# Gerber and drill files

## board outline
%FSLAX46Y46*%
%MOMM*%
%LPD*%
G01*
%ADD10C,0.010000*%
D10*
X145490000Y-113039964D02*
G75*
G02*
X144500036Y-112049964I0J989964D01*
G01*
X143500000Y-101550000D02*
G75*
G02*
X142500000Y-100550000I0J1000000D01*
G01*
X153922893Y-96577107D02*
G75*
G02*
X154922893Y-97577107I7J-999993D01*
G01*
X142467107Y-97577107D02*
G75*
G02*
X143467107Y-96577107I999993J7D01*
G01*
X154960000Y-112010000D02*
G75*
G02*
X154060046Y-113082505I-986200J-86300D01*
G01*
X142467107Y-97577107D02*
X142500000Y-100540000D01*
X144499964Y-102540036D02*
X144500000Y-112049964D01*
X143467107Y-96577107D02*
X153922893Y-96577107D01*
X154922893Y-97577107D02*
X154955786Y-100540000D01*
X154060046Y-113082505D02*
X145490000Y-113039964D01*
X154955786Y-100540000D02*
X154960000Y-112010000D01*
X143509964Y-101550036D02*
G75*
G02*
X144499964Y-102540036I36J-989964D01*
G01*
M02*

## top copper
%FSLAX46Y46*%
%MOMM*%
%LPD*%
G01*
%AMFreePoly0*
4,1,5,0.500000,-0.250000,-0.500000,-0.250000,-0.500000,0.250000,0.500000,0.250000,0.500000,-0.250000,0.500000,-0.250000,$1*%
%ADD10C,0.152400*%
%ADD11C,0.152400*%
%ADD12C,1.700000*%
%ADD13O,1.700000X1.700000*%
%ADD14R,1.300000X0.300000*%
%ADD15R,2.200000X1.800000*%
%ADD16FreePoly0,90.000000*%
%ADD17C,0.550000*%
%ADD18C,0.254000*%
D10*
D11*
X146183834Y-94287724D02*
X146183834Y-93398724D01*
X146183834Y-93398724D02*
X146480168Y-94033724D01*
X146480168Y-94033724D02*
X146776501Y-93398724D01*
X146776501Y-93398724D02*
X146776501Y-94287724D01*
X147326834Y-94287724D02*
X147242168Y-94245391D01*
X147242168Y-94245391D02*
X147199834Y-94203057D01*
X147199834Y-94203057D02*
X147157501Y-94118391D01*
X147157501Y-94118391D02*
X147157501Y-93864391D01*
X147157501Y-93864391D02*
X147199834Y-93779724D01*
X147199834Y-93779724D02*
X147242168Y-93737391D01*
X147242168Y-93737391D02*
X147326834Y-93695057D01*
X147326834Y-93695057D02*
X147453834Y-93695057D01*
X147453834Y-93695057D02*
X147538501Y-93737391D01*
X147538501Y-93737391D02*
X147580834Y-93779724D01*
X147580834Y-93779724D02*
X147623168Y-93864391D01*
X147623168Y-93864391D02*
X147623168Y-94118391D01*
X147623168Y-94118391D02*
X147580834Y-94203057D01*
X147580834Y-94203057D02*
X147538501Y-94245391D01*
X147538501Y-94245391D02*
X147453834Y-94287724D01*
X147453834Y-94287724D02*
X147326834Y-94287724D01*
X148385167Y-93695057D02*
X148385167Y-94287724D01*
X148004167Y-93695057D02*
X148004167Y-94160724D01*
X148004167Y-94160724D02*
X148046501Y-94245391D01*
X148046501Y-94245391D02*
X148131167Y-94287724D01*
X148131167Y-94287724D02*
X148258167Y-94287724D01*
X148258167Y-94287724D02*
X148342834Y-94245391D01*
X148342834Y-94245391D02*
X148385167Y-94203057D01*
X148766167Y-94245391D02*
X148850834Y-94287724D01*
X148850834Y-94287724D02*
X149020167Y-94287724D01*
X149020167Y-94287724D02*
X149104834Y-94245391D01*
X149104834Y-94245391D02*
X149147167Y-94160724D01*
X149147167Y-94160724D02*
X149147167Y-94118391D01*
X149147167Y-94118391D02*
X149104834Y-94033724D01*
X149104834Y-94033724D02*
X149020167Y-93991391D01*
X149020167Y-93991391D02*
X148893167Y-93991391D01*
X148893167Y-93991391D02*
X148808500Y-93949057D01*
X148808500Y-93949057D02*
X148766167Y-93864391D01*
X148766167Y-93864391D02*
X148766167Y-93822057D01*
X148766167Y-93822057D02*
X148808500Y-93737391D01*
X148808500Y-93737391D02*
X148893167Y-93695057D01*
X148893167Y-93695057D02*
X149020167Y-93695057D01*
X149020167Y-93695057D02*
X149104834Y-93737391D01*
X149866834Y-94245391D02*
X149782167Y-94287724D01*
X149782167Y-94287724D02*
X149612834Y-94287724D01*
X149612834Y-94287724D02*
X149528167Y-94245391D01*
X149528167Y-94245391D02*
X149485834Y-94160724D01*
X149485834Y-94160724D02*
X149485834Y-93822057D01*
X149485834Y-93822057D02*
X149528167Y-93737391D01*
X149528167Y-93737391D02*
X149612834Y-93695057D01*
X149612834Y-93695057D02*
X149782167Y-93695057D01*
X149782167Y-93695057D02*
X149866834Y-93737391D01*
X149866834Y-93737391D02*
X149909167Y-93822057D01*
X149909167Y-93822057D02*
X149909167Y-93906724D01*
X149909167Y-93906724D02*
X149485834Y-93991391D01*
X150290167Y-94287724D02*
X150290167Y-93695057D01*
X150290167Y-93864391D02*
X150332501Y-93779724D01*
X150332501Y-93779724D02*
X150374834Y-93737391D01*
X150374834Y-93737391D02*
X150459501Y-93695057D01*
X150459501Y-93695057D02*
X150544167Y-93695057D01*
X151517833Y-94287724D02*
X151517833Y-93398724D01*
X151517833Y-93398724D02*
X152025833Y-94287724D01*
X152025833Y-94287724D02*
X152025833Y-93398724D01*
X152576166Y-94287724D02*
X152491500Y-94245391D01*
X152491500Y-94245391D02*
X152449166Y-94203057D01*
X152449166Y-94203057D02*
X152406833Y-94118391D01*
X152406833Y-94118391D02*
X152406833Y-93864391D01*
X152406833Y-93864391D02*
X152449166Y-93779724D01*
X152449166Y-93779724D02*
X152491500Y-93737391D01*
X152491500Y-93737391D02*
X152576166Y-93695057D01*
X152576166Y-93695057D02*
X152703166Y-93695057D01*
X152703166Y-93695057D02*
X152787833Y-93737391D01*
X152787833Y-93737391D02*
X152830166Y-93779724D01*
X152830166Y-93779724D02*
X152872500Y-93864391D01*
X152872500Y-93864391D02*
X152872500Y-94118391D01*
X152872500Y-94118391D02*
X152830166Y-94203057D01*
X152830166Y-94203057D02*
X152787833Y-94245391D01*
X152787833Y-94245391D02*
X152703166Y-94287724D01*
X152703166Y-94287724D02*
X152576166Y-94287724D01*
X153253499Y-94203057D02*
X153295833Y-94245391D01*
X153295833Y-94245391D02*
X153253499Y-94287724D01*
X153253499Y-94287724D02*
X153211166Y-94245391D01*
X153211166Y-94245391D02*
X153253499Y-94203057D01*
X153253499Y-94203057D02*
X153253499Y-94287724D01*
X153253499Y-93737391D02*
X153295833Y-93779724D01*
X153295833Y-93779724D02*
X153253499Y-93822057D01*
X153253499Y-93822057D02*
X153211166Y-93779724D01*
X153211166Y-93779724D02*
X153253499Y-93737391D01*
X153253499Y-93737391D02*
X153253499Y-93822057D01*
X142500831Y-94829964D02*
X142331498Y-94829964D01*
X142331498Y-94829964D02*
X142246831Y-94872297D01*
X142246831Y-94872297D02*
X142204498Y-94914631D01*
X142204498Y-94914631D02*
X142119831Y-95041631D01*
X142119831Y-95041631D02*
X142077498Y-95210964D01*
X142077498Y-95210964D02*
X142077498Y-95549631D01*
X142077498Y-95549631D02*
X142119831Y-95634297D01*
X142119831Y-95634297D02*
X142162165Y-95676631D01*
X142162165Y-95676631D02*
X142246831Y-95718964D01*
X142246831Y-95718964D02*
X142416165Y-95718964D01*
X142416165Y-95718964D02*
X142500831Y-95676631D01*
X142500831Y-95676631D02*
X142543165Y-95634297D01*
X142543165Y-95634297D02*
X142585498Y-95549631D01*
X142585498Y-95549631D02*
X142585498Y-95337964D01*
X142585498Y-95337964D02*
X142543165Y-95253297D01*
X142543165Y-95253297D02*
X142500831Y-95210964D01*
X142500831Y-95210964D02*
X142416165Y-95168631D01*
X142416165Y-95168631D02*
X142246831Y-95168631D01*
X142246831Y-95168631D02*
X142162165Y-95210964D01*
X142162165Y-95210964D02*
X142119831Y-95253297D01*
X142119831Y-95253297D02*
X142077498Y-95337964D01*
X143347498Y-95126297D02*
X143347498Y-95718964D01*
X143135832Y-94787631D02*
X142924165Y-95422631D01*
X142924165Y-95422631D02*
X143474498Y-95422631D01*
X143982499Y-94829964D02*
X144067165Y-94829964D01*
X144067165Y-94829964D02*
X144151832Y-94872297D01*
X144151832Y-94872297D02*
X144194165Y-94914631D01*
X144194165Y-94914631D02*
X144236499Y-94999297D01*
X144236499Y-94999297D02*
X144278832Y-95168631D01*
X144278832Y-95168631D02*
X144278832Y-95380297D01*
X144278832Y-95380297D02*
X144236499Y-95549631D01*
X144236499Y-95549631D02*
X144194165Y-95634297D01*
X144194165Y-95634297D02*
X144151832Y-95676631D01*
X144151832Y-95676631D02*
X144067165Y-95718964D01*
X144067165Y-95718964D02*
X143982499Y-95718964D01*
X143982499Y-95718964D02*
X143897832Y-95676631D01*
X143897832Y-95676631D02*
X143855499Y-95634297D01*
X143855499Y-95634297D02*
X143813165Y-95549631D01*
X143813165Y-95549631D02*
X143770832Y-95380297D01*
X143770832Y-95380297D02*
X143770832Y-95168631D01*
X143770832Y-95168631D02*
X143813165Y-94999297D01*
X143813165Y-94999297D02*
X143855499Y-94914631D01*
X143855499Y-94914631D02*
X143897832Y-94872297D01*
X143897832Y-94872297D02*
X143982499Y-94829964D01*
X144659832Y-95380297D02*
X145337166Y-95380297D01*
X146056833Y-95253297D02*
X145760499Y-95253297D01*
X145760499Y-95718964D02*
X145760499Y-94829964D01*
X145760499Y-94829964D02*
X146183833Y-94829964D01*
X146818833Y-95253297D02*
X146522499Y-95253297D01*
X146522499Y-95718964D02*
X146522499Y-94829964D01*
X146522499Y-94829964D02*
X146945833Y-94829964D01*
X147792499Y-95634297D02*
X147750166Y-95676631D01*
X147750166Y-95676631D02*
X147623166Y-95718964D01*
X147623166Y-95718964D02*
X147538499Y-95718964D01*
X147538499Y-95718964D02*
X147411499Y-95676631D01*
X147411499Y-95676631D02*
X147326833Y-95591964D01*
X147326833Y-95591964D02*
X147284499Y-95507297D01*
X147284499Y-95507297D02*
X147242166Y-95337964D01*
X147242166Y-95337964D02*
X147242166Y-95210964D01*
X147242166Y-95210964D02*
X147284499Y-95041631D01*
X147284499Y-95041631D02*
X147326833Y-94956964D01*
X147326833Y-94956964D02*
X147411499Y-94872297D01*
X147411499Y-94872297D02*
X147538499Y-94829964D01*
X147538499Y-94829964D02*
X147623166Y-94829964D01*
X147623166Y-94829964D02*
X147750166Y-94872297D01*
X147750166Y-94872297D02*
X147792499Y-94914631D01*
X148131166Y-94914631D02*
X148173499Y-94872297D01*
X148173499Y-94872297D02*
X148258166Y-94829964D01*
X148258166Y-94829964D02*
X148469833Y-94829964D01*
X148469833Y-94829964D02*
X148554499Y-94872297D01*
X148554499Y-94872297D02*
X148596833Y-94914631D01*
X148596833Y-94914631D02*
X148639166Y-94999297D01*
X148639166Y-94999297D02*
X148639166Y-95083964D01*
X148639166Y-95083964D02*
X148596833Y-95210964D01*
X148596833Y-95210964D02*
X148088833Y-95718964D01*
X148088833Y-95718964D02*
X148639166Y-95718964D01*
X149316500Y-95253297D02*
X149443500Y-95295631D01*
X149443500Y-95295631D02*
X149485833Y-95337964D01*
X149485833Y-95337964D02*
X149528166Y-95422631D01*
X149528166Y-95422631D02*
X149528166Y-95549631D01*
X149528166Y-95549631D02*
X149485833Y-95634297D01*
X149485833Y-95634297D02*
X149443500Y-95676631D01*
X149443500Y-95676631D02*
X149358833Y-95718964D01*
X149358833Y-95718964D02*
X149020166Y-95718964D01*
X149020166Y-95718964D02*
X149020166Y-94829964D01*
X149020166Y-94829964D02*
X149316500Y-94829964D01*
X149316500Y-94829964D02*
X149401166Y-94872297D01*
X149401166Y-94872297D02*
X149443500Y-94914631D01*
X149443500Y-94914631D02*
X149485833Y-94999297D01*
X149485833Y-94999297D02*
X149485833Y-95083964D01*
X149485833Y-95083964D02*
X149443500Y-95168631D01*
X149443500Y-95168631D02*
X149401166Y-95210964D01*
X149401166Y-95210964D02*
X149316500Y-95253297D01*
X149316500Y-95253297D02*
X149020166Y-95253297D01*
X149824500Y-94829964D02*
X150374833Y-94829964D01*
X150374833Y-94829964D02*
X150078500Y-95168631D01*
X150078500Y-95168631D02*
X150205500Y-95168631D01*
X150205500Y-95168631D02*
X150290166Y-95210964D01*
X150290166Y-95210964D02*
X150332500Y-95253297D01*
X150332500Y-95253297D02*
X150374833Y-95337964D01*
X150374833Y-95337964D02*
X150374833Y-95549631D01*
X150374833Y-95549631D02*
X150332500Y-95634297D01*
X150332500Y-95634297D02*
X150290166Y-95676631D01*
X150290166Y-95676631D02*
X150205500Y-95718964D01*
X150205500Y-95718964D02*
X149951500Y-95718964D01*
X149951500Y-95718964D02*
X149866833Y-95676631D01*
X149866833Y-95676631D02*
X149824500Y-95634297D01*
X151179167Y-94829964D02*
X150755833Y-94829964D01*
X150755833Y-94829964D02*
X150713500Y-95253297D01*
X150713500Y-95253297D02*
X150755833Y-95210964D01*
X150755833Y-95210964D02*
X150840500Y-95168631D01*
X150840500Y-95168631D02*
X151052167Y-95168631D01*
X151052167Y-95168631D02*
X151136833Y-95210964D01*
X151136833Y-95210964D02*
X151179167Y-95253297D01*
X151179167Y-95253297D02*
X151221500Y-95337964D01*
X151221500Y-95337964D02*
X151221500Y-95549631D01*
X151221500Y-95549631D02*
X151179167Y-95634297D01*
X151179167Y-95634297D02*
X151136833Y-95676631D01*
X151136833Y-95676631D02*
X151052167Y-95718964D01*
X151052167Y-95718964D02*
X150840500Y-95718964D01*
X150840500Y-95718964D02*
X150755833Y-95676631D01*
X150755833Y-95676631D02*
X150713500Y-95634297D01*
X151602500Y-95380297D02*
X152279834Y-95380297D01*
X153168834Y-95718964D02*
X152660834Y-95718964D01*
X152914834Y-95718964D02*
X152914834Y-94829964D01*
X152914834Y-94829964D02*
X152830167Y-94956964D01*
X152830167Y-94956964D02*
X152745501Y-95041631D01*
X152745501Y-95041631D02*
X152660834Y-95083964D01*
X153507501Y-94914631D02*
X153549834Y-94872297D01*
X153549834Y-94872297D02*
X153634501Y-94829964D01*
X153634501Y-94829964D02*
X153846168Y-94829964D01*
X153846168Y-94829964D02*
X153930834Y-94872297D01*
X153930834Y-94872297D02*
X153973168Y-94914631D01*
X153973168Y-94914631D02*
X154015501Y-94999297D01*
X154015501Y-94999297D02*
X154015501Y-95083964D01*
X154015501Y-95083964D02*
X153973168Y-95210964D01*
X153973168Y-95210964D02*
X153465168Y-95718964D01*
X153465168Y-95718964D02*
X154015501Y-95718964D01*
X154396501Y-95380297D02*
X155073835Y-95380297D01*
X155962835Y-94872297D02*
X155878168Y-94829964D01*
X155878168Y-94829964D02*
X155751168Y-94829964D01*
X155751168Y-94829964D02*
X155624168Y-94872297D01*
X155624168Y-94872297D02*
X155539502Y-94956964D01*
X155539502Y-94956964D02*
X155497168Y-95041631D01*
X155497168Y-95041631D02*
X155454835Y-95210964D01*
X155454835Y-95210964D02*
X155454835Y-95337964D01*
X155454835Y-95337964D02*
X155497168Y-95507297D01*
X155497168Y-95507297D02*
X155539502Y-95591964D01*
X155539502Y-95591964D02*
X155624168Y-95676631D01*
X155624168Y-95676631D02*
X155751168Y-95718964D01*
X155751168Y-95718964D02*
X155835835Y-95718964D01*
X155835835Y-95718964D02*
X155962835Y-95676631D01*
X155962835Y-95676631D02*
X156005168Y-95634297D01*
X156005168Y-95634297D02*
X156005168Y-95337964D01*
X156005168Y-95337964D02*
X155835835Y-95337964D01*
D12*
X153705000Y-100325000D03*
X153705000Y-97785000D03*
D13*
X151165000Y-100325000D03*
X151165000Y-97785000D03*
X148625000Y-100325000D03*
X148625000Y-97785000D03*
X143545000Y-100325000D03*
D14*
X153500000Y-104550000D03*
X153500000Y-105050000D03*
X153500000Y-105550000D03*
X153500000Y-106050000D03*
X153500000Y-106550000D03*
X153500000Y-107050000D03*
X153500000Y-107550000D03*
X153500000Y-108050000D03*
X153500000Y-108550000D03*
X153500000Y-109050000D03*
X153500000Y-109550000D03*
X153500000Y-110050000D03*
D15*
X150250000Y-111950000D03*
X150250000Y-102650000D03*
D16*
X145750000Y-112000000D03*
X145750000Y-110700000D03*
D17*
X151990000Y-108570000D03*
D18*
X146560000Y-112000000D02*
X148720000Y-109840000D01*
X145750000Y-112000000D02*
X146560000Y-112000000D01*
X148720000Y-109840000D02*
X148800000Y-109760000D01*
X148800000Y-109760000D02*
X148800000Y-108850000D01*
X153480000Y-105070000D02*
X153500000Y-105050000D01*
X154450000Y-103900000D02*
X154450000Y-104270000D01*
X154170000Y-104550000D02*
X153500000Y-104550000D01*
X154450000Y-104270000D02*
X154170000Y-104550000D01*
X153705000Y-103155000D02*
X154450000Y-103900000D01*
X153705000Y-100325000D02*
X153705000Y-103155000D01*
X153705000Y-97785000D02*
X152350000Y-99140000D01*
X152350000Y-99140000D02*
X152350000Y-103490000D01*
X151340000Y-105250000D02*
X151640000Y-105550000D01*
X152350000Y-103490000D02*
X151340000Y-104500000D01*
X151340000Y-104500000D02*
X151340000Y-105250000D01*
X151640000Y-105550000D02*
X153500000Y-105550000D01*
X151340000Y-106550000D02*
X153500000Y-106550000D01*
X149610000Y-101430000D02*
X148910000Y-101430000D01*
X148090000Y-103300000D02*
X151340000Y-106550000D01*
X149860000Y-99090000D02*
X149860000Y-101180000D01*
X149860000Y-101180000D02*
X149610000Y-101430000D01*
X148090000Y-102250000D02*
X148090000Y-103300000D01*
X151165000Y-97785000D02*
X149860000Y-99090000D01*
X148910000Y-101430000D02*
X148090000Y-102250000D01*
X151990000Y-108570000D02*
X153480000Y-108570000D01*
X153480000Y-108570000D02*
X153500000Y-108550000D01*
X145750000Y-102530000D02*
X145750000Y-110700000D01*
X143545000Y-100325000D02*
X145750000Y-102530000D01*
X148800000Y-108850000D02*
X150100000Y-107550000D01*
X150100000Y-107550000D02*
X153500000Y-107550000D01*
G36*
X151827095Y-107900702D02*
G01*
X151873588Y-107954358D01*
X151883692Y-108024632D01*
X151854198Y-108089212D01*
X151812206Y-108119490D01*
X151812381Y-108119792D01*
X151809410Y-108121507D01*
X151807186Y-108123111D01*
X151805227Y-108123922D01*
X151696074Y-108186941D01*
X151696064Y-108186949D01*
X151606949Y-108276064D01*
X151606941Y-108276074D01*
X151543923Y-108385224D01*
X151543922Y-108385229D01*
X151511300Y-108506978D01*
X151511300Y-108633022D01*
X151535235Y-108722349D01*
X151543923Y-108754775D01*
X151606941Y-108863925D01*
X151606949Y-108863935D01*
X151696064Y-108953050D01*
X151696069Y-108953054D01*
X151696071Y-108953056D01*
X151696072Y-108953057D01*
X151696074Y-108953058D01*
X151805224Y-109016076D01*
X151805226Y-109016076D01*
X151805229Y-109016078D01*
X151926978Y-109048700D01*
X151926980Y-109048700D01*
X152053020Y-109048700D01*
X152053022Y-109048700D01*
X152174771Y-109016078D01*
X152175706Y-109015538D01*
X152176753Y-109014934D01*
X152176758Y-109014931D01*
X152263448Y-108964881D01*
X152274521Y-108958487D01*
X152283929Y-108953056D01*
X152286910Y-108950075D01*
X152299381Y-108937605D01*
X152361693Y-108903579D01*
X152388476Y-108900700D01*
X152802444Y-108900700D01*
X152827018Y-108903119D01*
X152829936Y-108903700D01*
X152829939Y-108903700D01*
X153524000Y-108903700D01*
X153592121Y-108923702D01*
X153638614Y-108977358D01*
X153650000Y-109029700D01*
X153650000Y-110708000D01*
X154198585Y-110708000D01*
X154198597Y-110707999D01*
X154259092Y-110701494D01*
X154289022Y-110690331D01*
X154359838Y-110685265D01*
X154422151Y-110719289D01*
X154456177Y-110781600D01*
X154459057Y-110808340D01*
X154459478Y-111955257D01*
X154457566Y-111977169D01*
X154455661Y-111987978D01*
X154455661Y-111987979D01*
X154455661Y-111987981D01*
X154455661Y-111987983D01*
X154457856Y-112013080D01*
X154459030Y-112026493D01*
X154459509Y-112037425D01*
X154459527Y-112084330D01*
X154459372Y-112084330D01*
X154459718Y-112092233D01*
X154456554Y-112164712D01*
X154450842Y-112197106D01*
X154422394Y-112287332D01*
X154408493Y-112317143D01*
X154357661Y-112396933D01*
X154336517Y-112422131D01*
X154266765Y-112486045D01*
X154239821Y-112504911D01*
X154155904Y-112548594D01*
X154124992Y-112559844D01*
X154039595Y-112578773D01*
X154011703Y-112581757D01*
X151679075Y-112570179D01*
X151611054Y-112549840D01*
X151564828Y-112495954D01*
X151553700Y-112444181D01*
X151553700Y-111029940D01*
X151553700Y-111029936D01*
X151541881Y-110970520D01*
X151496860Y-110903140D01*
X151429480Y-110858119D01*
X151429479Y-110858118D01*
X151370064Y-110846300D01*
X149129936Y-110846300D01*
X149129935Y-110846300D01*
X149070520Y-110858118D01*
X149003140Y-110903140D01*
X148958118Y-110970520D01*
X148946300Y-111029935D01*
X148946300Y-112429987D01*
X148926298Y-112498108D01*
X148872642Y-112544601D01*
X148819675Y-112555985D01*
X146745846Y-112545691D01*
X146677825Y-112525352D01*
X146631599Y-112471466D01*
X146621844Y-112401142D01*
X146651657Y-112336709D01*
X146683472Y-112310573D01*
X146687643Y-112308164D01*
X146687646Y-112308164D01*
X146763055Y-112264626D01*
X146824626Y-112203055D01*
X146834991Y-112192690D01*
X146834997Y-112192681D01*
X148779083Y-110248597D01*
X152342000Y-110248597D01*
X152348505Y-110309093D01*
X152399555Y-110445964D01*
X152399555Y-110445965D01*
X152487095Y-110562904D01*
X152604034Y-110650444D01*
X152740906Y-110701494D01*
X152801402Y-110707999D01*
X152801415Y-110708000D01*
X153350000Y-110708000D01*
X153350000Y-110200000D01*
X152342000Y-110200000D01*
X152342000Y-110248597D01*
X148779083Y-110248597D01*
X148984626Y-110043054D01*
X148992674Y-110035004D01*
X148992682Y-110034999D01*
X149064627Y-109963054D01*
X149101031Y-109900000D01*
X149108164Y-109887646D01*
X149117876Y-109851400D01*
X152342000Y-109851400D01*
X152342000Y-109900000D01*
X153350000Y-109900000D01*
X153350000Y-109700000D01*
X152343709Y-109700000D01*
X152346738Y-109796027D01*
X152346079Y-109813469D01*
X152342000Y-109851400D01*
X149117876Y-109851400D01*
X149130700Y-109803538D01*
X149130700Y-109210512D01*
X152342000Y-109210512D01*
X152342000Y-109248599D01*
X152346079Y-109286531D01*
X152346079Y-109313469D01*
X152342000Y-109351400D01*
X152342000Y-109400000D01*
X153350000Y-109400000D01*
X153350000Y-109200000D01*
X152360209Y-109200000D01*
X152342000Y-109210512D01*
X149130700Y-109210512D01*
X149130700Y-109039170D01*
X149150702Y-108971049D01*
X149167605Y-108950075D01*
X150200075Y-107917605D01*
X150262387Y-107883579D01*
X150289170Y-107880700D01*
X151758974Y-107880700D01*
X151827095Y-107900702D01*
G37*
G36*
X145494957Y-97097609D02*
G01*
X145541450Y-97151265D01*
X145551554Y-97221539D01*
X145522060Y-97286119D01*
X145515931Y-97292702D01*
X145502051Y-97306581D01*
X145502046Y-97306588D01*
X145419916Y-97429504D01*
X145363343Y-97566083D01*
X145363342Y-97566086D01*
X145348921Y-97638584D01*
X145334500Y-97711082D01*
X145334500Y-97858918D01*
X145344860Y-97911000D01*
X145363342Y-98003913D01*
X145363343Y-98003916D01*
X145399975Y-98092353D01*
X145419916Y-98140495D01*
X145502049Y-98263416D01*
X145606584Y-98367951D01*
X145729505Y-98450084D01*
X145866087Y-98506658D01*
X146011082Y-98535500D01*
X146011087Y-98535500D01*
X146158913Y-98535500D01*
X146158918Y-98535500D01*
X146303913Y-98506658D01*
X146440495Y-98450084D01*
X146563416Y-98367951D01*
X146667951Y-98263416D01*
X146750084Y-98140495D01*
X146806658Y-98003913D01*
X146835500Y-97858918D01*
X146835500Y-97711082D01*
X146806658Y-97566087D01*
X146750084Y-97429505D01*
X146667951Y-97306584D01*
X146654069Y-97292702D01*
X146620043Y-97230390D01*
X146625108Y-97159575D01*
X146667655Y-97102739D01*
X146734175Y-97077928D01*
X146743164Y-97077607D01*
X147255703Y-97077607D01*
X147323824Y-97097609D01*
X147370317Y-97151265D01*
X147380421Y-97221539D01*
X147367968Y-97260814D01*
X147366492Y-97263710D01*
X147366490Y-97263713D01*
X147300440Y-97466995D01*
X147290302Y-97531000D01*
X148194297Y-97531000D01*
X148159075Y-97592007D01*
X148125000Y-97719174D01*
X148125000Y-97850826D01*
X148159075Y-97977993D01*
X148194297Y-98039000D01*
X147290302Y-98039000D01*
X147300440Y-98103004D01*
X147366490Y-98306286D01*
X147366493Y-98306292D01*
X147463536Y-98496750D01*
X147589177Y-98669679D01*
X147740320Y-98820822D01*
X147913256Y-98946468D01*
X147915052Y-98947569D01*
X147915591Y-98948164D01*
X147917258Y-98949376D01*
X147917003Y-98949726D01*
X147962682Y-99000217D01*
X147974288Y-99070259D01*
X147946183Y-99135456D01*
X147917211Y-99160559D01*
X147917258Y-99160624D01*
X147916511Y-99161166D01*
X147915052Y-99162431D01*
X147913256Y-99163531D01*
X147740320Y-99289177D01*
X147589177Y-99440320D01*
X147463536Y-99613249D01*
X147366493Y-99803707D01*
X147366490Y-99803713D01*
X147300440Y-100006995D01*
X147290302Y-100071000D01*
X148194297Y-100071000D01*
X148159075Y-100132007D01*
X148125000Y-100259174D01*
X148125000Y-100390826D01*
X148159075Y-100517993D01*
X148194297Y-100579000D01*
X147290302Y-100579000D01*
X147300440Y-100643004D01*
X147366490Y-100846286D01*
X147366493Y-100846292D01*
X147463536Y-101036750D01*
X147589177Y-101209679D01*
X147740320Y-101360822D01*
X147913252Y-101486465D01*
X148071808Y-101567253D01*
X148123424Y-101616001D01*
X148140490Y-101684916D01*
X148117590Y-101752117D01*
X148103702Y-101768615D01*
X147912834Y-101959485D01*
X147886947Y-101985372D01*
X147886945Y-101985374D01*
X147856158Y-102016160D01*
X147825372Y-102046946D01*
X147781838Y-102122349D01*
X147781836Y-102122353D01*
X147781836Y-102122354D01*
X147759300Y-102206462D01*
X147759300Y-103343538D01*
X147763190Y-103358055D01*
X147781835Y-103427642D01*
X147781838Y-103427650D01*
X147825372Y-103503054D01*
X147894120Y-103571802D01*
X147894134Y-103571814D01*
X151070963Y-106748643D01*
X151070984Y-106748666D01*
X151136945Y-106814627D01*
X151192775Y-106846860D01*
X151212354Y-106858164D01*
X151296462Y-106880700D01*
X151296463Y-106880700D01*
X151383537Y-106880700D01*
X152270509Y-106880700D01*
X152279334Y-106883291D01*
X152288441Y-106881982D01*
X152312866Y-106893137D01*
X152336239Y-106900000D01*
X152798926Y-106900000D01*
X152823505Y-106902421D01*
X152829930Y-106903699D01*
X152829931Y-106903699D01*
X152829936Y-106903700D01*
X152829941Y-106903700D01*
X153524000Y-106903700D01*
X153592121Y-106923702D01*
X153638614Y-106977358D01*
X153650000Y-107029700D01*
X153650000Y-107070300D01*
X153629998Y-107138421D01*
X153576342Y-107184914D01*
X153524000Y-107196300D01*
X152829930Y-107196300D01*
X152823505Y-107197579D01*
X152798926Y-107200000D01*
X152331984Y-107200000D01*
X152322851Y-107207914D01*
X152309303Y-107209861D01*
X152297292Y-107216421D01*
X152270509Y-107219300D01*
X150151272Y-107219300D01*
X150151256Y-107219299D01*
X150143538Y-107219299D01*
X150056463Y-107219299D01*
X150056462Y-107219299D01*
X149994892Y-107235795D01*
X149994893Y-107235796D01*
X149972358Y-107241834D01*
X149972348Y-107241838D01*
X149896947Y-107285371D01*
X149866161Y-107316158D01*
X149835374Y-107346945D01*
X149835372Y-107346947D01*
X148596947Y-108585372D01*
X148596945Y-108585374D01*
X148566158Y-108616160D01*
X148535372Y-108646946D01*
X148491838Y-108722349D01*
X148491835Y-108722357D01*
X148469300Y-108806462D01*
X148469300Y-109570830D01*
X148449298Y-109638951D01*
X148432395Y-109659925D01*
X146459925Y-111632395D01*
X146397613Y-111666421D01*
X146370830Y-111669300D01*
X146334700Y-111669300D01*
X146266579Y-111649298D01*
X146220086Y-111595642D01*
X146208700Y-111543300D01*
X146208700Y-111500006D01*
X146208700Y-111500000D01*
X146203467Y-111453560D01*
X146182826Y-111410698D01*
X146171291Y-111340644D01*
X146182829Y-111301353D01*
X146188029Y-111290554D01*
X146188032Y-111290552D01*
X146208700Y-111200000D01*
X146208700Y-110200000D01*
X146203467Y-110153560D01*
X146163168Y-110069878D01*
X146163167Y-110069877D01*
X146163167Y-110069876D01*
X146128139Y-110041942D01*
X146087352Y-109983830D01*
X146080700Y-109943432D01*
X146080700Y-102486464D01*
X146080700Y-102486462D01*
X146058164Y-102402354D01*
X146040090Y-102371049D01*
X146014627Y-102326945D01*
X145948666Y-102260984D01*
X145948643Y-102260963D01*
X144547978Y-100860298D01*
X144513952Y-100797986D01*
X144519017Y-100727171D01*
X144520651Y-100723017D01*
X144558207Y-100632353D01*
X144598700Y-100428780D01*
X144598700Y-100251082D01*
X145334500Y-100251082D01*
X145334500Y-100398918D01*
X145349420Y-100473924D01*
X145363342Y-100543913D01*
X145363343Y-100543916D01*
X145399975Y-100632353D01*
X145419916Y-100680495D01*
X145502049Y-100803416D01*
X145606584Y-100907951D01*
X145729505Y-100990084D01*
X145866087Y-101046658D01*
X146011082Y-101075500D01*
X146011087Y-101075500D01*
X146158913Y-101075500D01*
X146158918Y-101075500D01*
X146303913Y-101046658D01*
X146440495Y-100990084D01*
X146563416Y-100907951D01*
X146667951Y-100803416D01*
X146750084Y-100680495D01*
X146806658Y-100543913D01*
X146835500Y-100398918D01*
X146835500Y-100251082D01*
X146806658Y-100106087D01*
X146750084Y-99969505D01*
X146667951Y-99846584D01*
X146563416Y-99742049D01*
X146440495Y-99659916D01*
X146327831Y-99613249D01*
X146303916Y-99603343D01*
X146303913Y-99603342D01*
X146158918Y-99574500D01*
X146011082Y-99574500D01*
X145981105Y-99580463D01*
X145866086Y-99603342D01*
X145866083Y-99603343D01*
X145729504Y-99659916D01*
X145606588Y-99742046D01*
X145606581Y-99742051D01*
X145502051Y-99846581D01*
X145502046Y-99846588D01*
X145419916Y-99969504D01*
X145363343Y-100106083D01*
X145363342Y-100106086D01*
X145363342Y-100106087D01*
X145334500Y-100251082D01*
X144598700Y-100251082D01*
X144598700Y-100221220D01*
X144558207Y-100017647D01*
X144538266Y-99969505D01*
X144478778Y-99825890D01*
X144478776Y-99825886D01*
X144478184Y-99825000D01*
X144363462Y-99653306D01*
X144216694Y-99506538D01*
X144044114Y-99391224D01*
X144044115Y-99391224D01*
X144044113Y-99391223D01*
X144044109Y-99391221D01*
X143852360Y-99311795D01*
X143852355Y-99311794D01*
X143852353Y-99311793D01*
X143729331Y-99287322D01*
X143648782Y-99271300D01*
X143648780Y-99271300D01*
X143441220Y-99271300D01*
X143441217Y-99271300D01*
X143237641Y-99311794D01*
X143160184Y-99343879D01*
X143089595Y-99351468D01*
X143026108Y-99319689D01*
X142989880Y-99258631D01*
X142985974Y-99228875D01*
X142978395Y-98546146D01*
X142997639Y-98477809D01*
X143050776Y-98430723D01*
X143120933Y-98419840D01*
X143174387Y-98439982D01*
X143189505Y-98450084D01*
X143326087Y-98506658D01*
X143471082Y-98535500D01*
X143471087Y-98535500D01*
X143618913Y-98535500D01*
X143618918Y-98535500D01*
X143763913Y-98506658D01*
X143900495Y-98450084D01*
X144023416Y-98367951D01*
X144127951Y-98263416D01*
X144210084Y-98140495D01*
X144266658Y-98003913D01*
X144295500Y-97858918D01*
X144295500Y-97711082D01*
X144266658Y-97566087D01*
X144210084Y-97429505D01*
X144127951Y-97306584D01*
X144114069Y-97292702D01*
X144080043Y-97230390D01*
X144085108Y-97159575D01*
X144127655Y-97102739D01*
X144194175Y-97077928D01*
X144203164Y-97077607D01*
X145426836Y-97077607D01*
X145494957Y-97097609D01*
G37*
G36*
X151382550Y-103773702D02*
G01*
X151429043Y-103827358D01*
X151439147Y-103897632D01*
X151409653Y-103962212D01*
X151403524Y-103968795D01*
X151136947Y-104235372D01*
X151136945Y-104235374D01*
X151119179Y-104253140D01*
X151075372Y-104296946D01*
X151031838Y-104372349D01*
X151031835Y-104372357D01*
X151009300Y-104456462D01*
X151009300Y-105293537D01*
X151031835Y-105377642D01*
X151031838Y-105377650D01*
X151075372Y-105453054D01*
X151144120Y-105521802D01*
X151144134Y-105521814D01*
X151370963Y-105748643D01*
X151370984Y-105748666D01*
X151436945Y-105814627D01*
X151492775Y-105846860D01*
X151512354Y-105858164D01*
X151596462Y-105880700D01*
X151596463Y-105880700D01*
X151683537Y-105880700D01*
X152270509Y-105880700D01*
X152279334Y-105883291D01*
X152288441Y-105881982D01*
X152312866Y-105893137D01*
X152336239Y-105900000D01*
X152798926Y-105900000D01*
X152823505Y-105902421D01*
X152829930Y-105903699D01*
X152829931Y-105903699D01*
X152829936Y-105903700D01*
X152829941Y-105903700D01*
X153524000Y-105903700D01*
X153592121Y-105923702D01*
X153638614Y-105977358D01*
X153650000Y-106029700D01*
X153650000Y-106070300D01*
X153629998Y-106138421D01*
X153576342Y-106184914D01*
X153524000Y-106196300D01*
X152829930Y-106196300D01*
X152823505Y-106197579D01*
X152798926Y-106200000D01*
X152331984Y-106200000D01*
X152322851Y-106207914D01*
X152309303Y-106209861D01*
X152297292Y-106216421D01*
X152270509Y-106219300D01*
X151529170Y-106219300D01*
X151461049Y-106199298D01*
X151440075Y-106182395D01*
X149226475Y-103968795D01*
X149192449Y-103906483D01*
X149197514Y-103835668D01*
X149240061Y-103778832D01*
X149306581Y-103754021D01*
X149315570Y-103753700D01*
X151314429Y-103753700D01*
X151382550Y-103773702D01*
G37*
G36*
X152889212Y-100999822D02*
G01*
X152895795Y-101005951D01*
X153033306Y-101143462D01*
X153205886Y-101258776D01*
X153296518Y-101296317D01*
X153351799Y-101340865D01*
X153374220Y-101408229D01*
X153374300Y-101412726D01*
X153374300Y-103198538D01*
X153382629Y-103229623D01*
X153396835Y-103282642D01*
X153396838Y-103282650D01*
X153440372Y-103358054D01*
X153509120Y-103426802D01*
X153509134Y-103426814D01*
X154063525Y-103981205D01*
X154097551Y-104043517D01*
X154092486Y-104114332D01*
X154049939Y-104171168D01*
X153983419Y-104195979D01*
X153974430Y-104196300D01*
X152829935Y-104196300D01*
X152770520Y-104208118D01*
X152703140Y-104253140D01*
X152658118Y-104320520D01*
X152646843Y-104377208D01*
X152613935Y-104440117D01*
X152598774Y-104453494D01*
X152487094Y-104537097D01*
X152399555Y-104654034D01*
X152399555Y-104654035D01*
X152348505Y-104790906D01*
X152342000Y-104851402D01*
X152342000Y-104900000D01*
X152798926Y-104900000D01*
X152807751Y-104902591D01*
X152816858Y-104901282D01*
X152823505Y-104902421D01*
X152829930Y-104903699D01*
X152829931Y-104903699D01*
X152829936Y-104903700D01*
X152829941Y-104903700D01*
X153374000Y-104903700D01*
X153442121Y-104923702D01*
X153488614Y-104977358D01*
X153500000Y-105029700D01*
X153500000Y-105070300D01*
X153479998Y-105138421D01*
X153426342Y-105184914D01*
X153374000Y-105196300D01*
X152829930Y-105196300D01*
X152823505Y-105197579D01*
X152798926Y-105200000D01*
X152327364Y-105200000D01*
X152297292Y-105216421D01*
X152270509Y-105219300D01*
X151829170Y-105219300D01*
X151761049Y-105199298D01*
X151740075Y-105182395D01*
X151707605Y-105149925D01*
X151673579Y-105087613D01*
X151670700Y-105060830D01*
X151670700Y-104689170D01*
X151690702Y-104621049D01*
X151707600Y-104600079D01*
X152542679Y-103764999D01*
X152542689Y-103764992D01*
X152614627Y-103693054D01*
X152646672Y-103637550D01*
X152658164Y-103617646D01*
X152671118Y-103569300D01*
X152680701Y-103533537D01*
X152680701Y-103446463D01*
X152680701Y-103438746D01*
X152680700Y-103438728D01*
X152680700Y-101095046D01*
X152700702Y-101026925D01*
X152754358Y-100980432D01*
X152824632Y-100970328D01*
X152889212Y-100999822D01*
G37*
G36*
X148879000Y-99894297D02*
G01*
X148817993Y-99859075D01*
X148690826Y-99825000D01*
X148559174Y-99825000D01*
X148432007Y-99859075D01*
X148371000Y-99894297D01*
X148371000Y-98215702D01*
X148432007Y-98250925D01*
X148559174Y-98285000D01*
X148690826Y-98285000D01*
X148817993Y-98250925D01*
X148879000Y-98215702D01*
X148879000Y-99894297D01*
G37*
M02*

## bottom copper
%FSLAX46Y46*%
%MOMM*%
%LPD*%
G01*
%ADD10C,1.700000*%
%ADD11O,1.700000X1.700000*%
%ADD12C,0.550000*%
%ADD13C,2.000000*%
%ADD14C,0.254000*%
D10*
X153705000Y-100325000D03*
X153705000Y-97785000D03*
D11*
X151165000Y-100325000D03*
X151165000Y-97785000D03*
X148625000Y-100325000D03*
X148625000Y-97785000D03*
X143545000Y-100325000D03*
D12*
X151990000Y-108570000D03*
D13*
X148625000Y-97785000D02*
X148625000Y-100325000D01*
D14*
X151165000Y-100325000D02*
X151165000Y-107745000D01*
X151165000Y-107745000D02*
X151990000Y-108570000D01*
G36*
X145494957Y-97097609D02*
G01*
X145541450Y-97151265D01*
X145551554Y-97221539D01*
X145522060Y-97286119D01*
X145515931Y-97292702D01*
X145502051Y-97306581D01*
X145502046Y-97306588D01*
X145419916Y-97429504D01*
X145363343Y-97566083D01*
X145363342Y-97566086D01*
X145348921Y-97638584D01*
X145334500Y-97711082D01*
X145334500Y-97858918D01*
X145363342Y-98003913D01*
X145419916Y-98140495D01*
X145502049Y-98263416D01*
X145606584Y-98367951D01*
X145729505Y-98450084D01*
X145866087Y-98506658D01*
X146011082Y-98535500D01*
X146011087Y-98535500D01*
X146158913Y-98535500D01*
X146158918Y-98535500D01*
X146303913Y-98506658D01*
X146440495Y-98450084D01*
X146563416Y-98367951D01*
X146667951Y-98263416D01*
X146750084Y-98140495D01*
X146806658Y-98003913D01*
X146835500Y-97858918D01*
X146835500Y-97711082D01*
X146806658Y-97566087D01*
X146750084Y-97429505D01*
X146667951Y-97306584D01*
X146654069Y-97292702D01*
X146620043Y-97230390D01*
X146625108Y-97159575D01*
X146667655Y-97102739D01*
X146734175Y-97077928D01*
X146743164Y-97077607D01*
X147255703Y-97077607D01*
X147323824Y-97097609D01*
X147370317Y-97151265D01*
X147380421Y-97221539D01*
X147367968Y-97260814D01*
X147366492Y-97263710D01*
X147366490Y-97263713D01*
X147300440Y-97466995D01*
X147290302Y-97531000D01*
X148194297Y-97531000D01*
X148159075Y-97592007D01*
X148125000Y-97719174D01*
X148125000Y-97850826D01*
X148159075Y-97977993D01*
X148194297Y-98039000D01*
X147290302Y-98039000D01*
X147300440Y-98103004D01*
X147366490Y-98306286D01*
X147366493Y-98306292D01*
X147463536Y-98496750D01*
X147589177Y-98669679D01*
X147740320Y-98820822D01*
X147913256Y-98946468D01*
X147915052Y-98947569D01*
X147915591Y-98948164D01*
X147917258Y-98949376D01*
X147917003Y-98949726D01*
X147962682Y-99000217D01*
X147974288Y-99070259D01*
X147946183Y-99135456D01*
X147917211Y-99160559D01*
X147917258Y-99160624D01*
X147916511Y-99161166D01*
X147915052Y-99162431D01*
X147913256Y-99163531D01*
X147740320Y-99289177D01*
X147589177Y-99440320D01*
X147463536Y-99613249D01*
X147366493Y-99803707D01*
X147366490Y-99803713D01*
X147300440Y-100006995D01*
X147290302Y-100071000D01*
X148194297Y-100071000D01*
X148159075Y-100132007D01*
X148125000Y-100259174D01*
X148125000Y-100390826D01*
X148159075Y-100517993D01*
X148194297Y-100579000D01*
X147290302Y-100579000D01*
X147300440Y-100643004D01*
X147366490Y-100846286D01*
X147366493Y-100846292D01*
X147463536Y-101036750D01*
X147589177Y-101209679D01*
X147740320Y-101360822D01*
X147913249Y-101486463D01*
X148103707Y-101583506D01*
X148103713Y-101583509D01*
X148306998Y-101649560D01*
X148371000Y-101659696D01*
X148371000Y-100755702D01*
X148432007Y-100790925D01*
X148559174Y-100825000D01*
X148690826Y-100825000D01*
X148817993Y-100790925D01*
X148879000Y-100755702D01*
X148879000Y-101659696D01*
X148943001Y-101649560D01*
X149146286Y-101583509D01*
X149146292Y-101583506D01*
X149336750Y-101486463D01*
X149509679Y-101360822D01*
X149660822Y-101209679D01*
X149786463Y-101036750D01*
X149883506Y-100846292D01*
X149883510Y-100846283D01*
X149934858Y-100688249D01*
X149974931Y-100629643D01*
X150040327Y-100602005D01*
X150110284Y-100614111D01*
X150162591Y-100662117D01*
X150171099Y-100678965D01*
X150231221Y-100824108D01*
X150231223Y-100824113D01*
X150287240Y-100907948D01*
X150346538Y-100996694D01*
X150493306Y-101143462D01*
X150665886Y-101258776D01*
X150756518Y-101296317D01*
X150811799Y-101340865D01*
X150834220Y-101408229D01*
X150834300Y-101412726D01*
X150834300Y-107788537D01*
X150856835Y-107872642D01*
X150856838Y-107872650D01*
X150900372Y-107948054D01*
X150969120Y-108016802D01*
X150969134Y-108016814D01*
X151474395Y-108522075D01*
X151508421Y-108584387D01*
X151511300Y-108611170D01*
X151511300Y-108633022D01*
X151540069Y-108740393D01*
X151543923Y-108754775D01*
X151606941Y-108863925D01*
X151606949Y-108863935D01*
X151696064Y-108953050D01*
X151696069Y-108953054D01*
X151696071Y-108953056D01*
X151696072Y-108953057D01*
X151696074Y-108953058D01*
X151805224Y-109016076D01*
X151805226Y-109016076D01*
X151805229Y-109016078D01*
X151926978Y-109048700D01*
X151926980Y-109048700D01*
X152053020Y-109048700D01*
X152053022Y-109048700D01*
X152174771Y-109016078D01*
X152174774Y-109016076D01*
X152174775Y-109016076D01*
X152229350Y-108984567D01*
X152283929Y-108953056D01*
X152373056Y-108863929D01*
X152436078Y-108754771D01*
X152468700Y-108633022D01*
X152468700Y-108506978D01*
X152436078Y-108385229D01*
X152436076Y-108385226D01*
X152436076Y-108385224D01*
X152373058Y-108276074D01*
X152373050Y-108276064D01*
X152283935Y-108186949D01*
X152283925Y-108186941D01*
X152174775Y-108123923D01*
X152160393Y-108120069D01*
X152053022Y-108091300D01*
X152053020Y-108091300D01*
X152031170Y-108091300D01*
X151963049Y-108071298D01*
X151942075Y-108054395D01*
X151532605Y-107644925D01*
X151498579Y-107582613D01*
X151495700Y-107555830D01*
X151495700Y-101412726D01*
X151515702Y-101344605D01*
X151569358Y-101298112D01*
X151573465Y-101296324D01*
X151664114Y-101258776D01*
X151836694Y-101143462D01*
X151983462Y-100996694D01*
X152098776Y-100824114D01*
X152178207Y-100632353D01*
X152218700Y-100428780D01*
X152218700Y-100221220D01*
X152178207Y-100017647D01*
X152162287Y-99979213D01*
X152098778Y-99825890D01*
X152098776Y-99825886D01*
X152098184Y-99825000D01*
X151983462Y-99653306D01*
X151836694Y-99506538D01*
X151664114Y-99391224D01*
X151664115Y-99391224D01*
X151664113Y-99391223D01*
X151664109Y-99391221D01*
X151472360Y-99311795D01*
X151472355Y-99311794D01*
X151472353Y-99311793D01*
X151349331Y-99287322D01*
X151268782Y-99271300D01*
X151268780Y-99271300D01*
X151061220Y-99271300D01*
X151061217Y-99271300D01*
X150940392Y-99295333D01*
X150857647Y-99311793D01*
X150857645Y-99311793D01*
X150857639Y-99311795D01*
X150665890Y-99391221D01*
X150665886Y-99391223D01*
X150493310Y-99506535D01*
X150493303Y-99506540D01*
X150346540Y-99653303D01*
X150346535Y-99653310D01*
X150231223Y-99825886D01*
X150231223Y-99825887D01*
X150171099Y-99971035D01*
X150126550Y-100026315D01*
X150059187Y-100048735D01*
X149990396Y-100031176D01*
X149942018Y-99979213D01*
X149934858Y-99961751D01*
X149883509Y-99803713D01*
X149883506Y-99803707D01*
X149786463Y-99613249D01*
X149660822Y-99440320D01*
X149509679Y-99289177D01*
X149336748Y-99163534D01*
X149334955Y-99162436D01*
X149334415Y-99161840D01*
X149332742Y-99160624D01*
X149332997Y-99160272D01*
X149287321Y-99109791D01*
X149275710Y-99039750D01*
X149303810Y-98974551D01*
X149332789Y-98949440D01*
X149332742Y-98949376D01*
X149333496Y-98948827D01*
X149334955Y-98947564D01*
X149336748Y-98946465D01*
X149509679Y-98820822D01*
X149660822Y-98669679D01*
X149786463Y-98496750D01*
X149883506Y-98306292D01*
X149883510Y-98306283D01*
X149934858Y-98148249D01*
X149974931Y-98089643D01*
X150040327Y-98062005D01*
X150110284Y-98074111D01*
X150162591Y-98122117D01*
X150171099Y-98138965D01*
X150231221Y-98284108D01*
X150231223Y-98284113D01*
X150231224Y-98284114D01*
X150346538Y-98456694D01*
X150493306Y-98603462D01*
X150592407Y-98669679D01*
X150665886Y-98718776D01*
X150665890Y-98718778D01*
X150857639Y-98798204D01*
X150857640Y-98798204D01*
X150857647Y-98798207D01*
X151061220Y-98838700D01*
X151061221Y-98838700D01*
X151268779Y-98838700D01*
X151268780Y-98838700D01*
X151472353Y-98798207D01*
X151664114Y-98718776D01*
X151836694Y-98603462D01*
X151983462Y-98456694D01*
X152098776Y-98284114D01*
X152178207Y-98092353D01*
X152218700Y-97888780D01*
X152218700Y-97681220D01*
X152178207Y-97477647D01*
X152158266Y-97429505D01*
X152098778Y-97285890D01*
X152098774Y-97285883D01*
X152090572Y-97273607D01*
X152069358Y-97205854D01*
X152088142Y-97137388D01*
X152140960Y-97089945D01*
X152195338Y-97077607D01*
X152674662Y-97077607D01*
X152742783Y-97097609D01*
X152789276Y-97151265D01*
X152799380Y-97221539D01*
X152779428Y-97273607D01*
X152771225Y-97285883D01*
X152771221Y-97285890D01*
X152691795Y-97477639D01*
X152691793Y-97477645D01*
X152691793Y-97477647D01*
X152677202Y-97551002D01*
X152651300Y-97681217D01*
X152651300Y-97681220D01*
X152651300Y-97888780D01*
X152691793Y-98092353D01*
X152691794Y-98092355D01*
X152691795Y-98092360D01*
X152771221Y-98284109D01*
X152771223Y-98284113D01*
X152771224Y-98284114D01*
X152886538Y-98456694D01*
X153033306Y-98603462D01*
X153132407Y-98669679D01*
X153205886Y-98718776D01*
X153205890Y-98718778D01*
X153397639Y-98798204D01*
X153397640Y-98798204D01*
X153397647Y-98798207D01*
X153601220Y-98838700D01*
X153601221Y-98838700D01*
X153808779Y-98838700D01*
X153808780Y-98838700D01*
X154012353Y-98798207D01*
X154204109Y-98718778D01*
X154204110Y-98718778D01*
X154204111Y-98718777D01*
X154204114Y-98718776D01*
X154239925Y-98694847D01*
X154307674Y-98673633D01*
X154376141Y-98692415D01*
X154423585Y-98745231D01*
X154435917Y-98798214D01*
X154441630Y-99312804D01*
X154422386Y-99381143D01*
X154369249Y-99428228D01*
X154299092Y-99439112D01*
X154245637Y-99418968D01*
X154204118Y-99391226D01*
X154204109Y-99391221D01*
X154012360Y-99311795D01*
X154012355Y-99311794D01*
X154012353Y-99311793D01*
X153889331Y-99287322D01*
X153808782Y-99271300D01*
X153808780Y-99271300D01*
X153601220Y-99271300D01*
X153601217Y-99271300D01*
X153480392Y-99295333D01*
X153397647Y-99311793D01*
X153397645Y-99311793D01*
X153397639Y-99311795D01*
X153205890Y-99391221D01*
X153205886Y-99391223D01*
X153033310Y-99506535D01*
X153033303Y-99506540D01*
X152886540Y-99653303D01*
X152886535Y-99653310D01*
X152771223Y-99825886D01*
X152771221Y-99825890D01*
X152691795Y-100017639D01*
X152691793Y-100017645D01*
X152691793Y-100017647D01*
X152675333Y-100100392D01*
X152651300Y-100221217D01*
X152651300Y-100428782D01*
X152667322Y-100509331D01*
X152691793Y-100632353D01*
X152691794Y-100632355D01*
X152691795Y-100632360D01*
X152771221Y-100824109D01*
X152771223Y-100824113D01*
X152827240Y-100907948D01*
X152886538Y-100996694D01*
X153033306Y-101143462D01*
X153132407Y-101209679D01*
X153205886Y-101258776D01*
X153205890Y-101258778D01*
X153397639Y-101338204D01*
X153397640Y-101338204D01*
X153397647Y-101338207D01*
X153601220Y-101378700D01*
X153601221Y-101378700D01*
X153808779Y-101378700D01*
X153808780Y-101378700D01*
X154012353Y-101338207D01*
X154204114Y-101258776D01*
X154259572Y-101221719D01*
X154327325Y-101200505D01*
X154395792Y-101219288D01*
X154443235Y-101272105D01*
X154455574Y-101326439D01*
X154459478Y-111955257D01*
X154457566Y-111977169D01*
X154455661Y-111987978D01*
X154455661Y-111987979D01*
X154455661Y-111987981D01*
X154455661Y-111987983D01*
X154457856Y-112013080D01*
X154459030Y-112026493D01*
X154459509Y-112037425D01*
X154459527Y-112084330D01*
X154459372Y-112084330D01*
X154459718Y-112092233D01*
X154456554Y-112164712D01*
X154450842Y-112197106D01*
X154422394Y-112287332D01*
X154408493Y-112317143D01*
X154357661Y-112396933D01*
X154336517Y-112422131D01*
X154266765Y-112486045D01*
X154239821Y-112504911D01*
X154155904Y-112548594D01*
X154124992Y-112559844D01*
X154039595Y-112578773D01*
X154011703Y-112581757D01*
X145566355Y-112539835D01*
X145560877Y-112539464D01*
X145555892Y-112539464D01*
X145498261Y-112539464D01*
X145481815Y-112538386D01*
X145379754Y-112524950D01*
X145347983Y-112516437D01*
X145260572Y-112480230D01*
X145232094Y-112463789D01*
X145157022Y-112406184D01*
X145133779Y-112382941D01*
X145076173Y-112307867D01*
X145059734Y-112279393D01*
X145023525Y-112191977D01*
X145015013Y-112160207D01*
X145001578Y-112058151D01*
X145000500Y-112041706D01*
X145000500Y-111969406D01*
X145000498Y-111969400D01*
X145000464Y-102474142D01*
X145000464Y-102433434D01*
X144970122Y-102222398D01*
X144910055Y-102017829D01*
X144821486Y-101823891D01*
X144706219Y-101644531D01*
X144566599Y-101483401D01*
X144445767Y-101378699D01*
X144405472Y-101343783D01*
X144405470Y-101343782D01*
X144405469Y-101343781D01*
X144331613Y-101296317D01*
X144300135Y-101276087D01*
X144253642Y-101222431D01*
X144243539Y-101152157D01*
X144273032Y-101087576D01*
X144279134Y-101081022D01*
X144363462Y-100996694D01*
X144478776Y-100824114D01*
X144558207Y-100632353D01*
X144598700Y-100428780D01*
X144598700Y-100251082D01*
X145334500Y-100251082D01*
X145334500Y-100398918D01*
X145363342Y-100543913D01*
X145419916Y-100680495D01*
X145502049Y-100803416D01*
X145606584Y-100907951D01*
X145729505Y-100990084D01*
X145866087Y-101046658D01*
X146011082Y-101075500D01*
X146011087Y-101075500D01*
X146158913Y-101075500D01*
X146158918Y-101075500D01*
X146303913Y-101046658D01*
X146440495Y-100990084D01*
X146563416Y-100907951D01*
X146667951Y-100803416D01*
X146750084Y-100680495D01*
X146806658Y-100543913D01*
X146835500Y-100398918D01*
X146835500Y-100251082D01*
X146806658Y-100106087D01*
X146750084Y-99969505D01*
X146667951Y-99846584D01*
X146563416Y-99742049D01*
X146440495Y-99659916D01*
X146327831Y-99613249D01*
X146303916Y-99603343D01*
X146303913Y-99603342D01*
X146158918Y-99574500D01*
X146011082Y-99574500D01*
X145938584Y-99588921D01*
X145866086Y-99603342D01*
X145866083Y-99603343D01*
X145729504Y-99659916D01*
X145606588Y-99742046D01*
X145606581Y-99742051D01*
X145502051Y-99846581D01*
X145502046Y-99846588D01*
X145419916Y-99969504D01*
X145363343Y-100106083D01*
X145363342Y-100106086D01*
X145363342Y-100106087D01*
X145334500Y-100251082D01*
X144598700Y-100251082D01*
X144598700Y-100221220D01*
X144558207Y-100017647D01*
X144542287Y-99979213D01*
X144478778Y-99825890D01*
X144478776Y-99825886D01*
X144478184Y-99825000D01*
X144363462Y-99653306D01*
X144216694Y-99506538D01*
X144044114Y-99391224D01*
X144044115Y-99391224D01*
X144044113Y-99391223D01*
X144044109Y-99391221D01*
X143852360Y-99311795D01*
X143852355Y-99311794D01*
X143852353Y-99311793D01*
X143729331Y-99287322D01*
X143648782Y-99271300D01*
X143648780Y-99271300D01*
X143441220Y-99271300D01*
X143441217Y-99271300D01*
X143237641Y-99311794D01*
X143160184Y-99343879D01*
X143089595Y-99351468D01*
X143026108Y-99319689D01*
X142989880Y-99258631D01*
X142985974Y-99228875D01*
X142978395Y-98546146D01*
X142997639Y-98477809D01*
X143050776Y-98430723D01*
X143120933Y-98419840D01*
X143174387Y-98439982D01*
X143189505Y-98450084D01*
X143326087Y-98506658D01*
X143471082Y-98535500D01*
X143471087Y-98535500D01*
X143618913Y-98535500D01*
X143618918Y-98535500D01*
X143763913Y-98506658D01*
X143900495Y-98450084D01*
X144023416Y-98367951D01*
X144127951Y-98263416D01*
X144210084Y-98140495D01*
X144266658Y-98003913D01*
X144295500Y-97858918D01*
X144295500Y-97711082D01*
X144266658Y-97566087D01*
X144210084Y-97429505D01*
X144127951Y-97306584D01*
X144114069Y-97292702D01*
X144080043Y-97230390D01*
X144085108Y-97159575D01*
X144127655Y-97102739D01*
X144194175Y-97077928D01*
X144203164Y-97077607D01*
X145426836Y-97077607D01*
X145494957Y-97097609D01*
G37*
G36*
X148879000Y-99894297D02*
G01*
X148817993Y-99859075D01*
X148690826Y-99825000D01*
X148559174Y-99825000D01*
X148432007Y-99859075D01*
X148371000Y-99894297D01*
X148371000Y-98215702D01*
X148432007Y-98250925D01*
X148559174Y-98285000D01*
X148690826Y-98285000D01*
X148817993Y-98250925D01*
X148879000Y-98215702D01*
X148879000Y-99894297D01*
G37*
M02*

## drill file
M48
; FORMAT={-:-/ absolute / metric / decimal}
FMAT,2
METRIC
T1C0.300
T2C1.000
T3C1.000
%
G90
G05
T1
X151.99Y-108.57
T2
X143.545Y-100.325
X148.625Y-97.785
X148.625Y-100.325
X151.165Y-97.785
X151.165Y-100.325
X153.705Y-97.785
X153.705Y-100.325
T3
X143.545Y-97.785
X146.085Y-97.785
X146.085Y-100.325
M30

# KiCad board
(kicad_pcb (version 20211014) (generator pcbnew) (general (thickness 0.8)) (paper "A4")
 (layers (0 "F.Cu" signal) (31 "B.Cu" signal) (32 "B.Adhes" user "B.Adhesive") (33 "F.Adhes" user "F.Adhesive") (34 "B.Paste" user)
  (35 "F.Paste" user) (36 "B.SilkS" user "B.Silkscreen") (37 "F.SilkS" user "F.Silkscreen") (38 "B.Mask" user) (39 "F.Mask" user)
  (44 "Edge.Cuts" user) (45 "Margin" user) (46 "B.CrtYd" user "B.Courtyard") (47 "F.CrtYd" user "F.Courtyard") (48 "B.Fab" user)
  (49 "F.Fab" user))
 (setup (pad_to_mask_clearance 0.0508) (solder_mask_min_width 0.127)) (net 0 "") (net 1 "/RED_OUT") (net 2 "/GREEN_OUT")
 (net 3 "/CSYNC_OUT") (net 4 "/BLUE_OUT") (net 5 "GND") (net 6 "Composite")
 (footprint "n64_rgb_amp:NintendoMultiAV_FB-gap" (layer "F.Cu") (at 147.355 99.055)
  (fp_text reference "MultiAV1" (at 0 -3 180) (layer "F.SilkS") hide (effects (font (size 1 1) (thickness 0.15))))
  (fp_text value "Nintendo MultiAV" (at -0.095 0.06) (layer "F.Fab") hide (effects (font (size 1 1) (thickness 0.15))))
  (pad "" np_thru_hole circle (at -1.27 -1.27) (size 1 1) (drill 1) (layers *.Cu *.Mask))
  (pad "" np_thru_hole circle (at -3.81 -1.27) (size 1 1) (drill 1) (layers *.Cu *.Mask))
  (pad "" np_thru_hole oval (at -1.27 1.27) (size 1 1) (drill 1) (layers *.Cu *.Mask))
  (pad "1" thru_hole circle (at 6.35 1.27) (size 1.7 1.7) (drill 1) (layers *.Cu *.Mask) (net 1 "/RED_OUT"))
  (pad "2" thru_hole circle (at 6.35 -1.27) (size 1.7 1.7) (drill 1) (layers *.Cu *.Mask) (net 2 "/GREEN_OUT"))
  (pad "3" thru_hole oval (at 3.81 1.27) (size 1.7 1.7) (drill 1) (layers *.Cu *.Mask) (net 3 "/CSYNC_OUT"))
  (pad "4" thru_hole oval (at 3.81 -1.27) (size 1.7 1.7) (drill 1) (layers *.Cu *.Mask) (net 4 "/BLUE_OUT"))
  (pad "5" thru_hole oval (at 1.27 1.27) (size 1.7 1.7) (drill 1) (layers *.Cu *.Mask) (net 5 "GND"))
  (pad "6" thru_hole oval (at 1.27 -1.27) (size 1.7 1.7) (drill 1) (layers *.Cu *.Mask) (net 5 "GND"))
  (pad "10" thru_hole oval (at -3.81 1.27) (size 1.7 1.7) (drill 1) (layers *.Cu *.Mask) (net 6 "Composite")))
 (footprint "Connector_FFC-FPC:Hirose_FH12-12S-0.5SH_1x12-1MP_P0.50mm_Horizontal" (layer "F.Cu") (at 151.65 107.3 -90)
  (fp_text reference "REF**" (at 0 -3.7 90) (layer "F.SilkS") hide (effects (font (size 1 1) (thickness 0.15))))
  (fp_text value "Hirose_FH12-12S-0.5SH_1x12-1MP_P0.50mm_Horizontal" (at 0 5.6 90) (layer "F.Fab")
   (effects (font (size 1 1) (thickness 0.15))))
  (pad "1" smd rect (at -2.75 -1.85 270) (size 0.3 1.3) (layers "F.Cu" "F.Paste" "F.Mask"))
  (pad "2" smd rect (at -2.25 -1.85 270) (size 0.3 1.3) (layers "F.Cu" "F.Paste" "F.Mask") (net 5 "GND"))
  (pad "3" smd rect (at -1.75 -1.85 270) (size 0.3 1.3) (layers "F.Cu" "F.Paste" "F.Mask"))
  (pad "4" smd rect (at -1.25 -1.85 270) (size 0.3 1.3) (layers "F.Cu" "F.Paste" "F.Mask") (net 5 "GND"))
  (pad "5" smd rect (at -0.75 -1.85 270) (size 0.3 1.3) (layers "F.Cu" "F.Paste" "F.Mask"))
  (pad "6" smd rect (at -0.25 -1.85 270) (size 0.3 1.3) (layers "F.Cu" "F.Paste" "F.Mask") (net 5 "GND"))
  (pad "7" smd rect (at 0.25 -1.85 270) (size 0.3 1.3) (layers "F.Cu" "F.Paste" "F.Mask"))
  (pad "8" smd rect (at 0.75 -1.85 270) (size 0.3 1.3) (layers "F.Cu" "F.Paste" "F.Mask") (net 5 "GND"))
  (pad "9" smd rect (at 1.25 -1.85 270) (size 0.3 1.3) (layers "F.Cu" "F.Paste" "F.Mask"))
  (pad "10" smd rect (at 1.75 -1.85 270) (size 0.3 1.3) (layers "F.Cu" "F.Paste" "F.Mask") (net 5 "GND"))
  (pad "11" smd rect (at 2.25 -1.85 270) (size 0.3 1.3) (layers "F.Cu" "F.Paste" "F.Mask") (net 5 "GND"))
  (pad "12" smd rect (at 2.75 -1.85 270) (size 0.3 1.3) (layers "F.Cu" "F.Paste" "F.Mask") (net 5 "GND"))
  (pad "MP" smd rect (at 4.65 1.4 270) (size 1.8 2.2) (layers "F.Cu" "F.Paste" "F.Mask"))
  (pad "MP" smd rect (at -4.65 1.4 270) (size 1.8 2.2) (layers "F.Cu" "F.Paste" "F.Mask")))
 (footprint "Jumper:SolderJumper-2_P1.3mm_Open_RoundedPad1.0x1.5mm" (layer "F.Cu") (at 145.75 111.35 90)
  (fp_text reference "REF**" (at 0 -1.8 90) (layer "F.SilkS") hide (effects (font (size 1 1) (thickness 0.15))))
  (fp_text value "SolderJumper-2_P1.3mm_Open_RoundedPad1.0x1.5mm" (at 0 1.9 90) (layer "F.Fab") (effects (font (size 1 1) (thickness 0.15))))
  (pad "1" smd custom (at -0.65 0 90) (size 1 0.5) (layers "F.Cu" "F.Mask") (zone_connect 2) (options (clearance outline) (anchor rect))
   (primitives))
  (pad "2" smd custom (at 0.65 0 90) (size 1 0.5) (layers "F.Cu" "F.Mask") (zone_connect 2) (options (clearance outline) (anchor rect))
   (primitives)))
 (gr_arc (start 145.49 113.039964) (mid 144.789964 112.75) (end 144.5 112.049964) (layer "Edge.Cuts") (width 0.01))
 (gr_arc (start 143.5 101.55) (mid 142.792893 101.257107) (end 142.5 100.55) (layer "Edge.Cuts") (width 0.01))
 (gr_arc (start 153.922893 96.577107) (mid 154.63 96.87) (end 154.922893 97.577107) (layer "Edge.Cuts") (width 0.01))
 (gr_arc (start 142.467107 97.577107) (mid 142.76 96.87) (end 143.467107 96.577107) (layer "Edge.Cuts") (width 0.01))
 (gr_arc (start 154.96 112.01) (mid 154.732149 112.732644) (end 154.060046 113.082505) (layer "Edge.Cuts") (width 0.01))
 (gr_line (start 142.467107 97.577107) (end 142.5 100.54) (layer "Edge.Cuts") (width 0.01))
 (gr_line (start 144.499964 102.540036) (end 144.5 112.049964) (layer "Edge.Cuts") (width 0.01))
 (gr_line (start 143.467107 96.577107) (end 153.922893 96.577107) (layer "Edge.Cuts") (width 0.01))
 (gr_line (start 154.922893 97.577107) (end 154.955786 100.54) (layer "Edge.Cuts") (width 0.01))
 (gr_line (start 154.060046 113.082505) (end 145.49 113.039964) (layer "Edge.Cuts") (width 0.01))
 (gr_line (start 154.955786 100.54) (end 154.96 112.01) (layer "Edge.Cuts") (width 0.01))
 (gr_arc (start 143.509964 101.550036) (mid 144.21 101.84) (end 144.499964 102.540036) (layer "Edge.Cuts") (width 0.01))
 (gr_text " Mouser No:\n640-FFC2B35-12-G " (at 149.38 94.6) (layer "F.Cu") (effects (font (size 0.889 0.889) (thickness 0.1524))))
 (segment (start 146.56 112) (end 148.72 109.84) (width 0.254) (layer "F.Cu") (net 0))
 (segment (start 145.75 112) (end 146.56 112) (width 0.254) (layer "F.Cu") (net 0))
 (segment (start 148.72 109.84) (end 148.8 109.76) (width 0.254) (layer "F.Cu") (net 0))
 (segment (start 148.8 109.76) (end 148.8 108.85) (width 0.254) (layer "F.Cu") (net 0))
 (segment (start 153.48 105.07) (end 153.5 105.05) (width 0.254) (layer "F.Cu") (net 5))
 (segment (start 148.625 97.785) (end 148.625 100.325) (width 2) (layer "B.Cu") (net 5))
 (segment (start 154.45 103.9) (end 154.45 104.27) (width 0.254) (layer "F.Cu") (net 1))
 (segment (start 154.17 104.55) (end 153.5 104.55) (width 0.254) (layer "F.Cu") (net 1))
 (segment (start 154.45 104.27) (end 154.17 104.55) (width 0.254) (layer "F.Cu") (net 1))
 (segment (start 153.705 103.155) (end 154.45 103.9) (width 0.254) (layer "F.Cu") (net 1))
 (segment (start 153.705 100.325) (end 153.705 103.155) (width 0.254) (layer "F.Cu") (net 1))
 (segment (start 153.705 97.785) (end 152.35 99.14) (width 0.254) (layer "F.Cu") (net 2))
 (segment (start 152.35 99.14) (end 152.35 103.49) (width 0.254) (layer "F.Cu") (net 2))
 (segment (start 151.34 105.25) (end 151.64 105.55) (width 0.254) (layer "F.Cu") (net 2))
 (segment (start 152.35 103.49) (end 151.34 104.5) (width 0.254) (layer "F.Cu") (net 2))
 (segment (start 151.34 104.5) (end 151.34 105.25) (width 0.254) (layer "F.Cu") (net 2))
 (segment (start 151.64 105.55) (end 153.5 105.55) (width 0.254) (layer "F.Cu") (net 2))
 (segment (start 151.34 106.55) (end 153.5 106.55) (width 0.254) (layer "F.Cu") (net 4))
 (segment (start 149.61 101.43) (end 148.91 101.43) (width 0.254) (layer "F.Cu") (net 4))
 (segment (start 148.09 103.3) (end 151.34 106.55) (width 0.254) (layer "F.Cu") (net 4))
 (segment (start 149.86 99.09) (end 149.86 101.18) (width 0.254) (layer "F.Cu") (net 4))
 (segment (start 149.86 101.18) (end 149.61 101.43) (width 0.254) (layer "F.Cu") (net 4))
 (segment (start 148.09 102.25) (end 148.09 103.3) (width 0.254) (layer "F.Cu") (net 4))
 (segment (start 151.165 97.785) (end 149.86 99.09) (width 0.254) (layer "F.Cu") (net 4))
 (segment (start 148.91 101.43) (end 148.09 102.25) (width 0.254) (layer "F.Cu") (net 4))
 (segment (start 151.99 108.57) (end 153.48 108.57) (width 0.254) (layer "F.Cu") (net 3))
 (segment (start 153.48 108.57) (end 153.5 108.55) (width 0.254) (layer "F.Cu") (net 3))
 (via (at 151.99 108.57) (size 0.55) (drill 0.3) (layers "F.Cu" "B.Cu") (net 3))
 (segment (start 151.165 100.325) (end 151.165 107.745) (width 0.254) (layer "B.Cu") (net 3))
 (segment (start 151.165 107.745) (end 151.99 108.57) (width 0.254) (layer "B.Cu") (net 3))
 (segment (start 145.75 102.53) (end 145.75 110.7) (width 0.254) (layer "F.Cu") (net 6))
 (segment (start 143.545 100.325) (end 145.75 102.53) (width 0.254) (layer "F.Cu") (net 6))
 (segment (start 148.8 108.85) (end 150.1 107.55) (width 0.254) (layer "F.Cu") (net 6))
 (segment (start 150.1 107.55) (end 153.5 107.55) (width 0.254) (layer "F.Cu") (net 6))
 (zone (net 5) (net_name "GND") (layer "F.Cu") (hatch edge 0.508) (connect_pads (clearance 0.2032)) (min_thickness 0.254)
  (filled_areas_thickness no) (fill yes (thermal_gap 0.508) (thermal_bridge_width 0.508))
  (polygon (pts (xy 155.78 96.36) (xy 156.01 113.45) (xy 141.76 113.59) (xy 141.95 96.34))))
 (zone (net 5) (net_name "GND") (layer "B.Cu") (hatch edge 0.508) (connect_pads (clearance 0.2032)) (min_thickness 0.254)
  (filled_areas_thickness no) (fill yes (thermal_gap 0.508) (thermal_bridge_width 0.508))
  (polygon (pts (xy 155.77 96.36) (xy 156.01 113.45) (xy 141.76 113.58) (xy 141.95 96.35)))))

